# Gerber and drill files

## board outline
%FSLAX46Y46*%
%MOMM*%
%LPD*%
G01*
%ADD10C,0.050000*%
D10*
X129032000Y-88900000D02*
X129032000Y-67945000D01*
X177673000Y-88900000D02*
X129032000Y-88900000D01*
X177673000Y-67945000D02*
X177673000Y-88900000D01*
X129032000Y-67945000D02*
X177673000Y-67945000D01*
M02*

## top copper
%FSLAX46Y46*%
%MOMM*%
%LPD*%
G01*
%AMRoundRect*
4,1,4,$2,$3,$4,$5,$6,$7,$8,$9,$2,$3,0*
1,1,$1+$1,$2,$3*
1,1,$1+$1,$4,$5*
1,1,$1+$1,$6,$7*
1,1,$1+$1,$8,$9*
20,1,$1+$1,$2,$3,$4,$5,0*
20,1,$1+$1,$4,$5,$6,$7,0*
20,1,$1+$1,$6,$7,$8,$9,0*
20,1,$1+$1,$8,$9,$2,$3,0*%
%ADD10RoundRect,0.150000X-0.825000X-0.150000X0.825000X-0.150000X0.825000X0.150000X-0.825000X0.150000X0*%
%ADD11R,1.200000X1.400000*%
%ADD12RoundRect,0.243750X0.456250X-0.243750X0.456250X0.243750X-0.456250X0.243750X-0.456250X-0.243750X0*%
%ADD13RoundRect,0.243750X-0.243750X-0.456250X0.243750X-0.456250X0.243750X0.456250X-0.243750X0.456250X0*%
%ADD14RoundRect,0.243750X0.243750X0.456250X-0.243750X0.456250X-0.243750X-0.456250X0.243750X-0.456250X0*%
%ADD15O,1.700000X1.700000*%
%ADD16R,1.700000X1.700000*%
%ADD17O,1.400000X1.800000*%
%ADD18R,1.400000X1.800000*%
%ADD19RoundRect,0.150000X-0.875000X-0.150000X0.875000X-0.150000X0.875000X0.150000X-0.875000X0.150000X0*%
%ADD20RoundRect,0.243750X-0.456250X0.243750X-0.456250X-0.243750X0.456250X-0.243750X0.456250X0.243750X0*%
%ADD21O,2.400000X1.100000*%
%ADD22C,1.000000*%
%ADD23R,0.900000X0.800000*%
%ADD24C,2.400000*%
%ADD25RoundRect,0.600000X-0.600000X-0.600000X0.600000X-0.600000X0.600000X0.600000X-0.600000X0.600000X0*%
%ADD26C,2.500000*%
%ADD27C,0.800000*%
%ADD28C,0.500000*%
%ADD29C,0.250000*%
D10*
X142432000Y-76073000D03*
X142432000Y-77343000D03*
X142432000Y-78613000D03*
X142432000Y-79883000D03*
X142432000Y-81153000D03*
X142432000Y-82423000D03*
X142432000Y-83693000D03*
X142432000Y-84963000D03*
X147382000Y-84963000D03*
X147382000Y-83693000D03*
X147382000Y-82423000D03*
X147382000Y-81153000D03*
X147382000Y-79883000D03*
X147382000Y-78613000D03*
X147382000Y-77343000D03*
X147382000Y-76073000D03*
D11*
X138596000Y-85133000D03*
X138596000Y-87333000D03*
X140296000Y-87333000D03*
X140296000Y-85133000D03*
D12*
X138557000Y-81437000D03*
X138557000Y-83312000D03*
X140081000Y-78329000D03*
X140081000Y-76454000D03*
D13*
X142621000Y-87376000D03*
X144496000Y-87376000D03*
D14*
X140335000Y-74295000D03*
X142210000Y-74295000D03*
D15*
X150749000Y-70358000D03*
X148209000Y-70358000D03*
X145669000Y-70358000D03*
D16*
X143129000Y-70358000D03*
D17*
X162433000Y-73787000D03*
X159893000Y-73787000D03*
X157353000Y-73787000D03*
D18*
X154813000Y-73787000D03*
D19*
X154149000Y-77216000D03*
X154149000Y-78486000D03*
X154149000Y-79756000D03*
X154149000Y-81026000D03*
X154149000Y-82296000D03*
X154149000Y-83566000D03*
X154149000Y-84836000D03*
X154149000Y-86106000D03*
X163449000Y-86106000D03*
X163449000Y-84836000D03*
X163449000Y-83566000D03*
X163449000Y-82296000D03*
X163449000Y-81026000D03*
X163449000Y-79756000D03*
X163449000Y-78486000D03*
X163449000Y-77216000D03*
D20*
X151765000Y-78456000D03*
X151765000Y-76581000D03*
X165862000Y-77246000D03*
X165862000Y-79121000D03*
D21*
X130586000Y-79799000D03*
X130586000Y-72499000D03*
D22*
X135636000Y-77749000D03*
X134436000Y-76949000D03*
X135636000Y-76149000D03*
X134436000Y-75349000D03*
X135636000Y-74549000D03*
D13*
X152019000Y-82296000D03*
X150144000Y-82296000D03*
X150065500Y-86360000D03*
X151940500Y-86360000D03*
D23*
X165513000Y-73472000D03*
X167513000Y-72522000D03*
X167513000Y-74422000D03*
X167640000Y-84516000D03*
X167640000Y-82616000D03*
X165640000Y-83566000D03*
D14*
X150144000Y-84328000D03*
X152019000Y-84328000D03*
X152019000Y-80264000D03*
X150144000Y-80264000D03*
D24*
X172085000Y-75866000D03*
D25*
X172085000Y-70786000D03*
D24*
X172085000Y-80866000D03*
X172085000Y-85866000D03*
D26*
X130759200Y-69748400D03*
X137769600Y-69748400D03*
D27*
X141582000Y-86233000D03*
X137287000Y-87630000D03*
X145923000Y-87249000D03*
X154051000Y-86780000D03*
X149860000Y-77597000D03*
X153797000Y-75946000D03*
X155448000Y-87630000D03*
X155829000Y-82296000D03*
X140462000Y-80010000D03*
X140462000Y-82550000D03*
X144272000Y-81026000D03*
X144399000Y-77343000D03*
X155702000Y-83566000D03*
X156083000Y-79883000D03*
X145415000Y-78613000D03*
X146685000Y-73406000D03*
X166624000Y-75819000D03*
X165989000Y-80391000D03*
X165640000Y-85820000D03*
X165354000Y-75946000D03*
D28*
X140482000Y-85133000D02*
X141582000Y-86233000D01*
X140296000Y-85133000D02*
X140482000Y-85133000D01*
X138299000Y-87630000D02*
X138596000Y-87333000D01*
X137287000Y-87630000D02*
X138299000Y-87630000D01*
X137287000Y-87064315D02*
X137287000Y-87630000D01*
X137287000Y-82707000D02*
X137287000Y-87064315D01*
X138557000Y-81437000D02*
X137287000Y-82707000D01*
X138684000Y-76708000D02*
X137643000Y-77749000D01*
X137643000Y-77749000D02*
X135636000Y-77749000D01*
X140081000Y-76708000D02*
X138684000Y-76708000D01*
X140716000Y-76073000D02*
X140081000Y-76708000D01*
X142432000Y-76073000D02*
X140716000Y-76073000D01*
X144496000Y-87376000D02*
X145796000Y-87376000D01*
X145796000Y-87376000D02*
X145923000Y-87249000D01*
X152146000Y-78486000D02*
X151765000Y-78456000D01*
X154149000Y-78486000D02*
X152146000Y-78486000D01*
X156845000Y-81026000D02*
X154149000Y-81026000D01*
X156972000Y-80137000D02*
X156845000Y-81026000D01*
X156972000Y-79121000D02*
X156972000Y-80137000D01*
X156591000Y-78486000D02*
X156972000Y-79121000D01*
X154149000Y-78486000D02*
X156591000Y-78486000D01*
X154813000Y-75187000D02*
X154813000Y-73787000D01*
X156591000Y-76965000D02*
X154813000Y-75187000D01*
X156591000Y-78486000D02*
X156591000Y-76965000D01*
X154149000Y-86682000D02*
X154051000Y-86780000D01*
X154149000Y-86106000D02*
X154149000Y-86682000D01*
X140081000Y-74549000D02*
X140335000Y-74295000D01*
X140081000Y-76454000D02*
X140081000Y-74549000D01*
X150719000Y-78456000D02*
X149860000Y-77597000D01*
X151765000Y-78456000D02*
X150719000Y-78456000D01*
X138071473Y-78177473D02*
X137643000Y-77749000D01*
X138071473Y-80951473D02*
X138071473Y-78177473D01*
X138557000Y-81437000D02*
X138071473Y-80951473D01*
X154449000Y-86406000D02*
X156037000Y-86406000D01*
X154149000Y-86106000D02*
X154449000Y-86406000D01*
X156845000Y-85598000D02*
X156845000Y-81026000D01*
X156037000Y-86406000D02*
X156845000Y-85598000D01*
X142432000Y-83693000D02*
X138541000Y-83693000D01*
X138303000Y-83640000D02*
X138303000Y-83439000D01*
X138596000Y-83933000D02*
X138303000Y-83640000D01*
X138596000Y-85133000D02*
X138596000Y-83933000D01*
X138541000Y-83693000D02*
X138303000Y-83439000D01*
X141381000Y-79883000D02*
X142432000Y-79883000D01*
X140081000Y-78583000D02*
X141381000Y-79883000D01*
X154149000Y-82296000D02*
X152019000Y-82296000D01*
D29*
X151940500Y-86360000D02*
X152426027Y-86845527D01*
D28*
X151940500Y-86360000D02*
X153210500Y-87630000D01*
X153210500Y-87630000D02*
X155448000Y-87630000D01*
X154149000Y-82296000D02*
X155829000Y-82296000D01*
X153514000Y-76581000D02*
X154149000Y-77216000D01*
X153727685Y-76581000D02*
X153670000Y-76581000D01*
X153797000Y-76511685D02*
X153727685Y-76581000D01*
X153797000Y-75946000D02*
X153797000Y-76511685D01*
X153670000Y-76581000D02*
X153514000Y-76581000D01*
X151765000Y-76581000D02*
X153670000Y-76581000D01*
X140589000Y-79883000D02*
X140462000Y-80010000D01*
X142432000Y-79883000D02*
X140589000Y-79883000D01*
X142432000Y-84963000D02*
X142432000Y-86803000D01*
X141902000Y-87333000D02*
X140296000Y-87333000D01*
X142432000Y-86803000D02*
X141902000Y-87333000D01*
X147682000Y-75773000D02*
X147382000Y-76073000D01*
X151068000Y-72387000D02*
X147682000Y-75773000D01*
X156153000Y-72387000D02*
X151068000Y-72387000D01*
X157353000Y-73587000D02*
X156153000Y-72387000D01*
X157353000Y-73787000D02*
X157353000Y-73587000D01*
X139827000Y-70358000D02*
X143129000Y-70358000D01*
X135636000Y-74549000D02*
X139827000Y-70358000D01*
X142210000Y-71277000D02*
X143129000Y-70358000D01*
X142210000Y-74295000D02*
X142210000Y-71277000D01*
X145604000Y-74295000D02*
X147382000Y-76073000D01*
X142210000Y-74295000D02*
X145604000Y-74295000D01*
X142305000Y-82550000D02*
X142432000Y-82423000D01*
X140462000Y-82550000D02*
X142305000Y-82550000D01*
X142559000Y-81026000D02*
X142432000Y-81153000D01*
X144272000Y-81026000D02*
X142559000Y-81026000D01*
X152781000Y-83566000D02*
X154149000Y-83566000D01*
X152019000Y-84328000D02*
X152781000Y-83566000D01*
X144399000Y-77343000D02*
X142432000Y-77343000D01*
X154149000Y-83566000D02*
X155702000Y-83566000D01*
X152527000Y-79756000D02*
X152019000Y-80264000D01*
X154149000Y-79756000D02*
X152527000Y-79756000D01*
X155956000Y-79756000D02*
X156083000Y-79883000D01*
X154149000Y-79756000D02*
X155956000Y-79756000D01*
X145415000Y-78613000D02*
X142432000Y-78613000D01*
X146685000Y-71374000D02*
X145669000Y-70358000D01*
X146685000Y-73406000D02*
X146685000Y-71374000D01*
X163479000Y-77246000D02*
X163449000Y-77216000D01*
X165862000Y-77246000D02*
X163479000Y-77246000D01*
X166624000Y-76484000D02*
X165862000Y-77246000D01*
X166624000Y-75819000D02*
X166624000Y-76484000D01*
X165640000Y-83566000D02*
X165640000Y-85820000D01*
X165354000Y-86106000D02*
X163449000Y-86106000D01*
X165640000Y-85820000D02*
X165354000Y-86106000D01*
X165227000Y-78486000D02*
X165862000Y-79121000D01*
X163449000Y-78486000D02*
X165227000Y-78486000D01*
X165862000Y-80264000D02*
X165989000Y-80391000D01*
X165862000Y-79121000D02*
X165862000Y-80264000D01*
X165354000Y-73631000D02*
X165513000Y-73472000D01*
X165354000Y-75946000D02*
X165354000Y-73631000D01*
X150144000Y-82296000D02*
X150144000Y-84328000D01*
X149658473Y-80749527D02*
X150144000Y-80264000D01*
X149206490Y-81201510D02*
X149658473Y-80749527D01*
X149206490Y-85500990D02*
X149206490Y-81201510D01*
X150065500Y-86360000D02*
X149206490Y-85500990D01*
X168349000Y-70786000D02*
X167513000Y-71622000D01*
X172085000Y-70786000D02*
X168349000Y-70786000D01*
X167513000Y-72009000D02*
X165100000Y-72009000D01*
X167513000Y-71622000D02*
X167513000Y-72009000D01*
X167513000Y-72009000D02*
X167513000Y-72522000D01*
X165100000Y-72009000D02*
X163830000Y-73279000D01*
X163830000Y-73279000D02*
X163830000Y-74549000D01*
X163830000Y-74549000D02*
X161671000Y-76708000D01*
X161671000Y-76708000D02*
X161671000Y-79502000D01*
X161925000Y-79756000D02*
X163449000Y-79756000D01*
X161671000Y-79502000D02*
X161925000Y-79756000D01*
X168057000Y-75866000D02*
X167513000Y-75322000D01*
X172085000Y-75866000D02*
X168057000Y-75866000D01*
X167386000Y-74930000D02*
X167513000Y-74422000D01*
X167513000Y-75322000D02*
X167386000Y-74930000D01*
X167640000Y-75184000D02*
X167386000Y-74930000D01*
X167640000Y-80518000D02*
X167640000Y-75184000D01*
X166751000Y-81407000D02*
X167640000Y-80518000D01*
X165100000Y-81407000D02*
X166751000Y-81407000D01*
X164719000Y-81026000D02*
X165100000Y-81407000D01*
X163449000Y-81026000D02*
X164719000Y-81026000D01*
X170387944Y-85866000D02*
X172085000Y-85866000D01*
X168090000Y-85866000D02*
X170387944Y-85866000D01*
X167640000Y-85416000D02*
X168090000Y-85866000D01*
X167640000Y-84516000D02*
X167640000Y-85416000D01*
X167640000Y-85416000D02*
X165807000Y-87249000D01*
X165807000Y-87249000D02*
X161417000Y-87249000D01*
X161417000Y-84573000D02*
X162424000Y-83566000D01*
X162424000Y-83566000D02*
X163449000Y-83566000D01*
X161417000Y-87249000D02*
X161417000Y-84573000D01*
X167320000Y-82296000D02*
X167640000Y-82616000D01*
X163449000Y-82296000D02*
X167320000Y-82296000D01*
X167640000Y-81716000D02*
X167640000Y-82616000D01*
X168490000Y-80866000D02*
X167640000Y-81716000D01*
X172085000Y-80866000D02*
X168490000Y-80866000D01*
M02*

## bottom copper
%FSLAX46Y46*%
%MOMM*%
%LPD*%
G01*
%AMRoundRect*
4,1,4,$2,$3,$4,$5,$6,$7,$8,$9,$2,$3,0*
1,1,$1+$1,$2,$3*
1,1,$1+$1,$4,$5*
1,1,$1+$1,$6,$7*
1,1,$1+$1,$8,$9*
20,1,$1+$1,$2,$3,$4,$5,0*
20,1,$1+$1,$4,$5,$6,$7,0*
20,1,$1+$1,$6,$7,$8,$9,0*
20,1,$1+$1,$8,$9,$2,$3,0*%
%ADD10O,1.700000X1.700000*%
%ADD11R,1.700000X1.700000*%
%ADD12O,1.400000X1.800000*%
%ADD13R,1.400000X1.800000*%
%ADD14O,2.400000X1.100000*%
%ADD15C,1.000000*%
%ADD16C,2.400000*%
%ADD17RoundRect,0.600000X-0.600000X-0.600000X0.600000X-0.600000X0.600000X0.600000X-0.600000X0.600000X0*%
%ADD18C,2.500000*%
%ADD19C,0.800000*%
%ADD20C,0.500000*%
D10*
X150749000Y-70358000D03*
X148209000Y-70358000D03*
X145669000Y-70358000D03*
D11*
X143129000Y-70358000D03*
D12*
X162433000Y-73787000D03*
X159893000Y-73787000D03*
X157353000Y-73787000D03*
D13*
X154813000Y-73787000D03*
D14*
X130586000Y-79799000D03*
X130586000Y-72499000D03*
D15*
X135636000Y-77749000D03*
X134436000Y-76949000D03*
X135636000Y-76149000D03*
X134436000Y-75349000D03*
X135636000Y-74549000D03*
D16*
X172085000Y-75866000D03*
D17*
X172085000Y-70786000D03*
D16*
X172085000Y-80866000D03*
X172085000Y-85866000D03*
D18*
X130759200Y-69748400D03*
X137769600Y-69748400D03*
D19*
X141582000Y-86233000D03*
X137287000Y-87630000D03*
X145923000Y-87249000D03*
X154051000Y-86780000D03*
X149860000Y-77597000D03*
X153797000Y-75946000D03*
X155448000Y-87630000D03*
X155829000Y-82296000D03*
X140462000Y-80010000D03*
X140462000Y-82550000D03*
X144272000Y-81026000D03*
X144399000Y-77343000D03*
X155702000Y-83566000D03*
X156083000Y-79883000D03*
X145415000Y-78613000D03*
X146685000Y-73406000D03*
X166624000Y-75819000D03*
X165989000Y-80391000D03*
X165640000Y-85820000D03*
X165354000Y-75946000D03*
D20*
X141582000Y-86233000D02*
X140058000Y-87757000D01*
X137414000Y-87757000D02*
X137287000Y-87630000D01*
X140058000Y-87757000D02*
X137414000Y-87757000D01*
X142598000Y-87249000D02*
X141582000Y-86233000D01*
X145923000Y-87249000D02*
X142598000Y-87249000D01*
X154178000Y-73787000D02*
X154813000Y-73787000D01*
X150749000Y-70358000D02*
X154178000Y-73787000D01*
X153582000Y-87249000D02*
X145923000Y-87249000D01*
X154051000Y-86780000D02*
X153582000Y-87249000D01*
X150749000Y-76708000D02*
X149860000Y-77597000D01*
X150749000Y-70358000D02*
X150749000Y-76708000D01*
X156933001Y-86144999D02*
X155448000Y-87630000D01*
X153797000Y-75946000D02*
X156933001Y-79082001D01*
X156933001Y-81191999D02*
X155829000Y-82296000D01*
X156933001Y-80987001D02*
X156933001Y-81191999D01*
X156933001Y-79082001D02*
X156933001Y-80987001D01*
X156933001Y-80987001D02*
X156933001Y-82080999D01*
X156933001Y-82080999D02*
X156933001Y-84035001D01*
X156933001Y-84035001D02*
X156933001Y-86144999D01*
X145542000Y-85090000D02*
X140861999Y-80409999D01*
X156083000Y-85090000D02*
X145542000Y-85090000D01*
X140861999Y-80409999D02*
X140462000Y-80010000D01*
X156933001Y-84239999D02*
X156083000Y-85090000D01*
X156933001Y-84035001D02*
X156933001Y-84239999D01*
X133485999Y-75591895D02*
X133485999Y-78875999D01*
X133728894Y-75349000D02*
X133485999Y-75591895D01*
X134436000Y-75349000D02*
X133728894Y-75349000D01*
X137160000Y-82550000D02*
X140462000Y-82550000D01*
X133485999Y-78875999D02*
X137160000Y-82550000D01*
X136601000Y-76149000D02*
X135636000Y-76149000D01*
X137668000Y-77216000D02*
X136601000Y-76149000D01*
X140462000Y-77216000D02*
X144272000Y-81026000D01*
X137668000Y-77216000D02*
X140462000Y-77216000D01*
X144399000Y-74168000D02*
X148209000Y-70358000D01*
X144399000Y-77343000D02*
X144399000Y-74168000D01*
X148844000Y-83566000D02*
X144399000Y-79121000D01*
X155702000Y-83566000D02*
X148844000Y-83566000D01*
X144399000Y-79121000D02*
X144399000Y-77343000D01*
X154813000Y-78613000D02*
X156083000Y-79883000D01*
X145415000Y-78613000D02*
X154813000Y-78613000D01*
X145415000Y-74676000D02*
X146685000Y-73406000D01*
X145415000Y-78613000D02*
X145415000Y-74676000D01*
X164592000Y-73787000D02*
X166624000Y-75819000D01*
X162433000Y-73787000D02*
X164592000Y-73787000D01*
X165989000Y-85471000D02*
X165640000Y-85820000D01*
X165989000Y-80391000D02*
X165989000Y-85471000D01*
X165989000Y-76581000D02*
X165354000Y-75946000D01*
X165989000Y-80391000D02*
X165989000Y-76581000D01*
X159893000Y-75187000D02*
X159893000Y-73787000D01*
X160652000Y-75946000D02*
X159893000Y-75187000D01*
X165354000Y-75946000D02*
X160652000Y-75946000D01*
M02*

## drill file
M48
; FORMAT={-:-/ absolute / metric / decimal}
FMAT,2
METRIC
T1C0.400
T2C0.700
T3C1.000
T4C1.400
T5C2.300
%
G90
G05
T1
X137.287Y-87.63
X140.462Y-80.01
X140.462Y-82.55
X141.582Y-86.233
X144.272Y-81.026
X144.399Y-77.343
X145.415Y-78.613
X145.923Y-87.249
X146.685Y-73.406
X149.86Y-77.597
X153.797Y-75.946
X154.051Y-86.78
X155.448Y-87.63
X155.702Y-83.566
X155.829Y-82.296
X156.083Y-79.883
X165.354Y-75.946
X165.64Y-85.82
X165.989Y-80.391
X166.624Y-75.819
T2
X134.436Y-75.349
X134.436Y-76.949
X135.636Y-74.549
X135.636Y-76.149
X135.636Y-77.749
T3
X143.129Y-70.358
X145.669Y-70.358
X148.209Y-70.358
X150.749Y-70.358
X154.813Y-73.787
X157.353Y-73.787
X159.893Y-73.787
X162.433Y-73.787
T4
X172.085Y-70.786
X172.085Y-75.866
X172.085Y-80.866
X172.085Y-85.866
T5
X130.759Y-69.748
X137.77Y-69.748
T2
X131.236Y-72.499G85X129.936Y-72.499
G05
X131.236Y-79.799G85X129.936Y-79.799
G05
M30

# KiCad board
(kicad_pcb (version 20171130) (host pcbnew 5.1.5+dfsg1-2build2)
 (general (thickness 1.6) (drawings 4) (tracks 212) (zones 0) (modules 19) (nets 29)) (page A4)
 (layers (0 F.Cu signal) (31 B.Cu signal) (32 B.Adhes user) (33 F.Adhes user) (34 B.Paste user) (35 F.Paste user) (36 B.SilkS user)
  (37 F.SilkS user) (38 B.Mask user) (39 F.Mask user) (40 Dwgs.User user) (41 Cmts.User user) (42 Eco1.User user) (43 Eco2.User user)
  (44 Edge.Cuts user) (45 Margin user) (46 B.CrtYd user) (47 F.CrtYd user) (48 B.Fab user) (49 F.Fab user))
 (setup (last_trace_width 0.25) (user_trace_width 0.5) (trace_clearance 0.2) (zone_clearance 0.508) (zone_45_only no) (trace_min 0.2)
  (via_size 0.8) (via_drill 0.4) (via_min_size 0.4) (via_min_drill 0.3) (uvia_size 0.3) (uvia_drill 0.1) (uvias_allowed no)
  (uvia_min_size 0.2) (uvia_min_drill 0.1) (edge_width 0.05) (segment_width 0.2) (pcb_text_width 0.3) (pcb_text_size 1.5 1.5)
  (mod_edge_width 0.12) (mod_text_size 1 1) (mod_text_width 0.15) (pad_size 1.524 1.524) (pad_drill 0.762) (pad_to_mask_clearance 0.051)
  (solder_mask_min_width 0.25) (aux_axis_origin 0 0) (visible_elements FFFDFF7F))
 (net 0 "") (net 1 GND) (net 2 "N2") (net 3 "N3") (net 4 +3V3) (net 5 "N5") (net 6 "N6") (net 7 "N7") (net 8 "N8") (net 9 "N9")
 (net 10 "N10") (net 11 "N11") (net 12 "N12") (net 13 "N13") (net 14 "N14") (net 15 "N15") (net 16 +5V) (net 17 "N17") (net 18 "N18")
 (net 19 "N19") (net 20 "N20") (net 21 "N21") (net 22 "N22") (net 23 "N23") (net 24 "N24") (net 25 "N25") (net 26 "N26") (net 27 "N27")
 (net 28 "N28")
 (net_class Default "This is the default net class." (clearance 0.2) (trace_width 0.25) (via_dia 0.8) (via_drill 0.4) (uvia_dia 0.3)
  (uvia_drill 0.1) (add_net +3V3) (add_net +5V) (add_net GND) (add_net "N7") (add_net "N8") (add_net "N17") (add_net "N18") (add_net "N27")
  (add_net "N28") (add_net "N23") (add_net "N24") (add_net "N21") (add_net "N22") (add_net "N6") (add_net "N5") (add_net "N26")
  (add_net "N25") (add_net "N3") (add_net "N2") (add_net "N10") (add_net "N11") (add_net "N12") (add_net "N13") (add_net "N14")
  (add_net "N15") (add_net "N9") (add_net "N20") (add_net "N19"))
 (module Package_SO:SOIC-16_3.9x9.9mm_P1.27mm (layer F.Cu) (at 144.907 80.518)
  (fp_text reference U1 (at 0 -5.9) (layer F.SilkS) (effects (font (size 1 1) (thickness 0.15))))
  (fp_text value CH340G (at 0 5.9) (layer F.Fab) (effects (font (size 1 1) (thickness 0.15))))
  (pad 1 smd roundrect (at -2.475 -4.445) (size 1.95 0.6) (layers F.Cu F.Paste F.Mask) (roundrect_rratio 0.25) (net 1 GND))
  (pad 2 smd roundrect (at -2.475 -3.175) (size 1.95 0.6) (layers F.Cu F.Paste F.Mask) (roundrect_rratio 0.25) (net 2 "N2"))
  (pad 3 smd roundrect (at -2.475 -1.905) (size 1.95 0.6) (layers F.Cu F.Paste F.Mask) (roundrect_rratio 0.25) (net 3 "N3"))
  (pad 4 smd roundrect (at -2.475 -0.635) (size 1.95 0.6) (layers F.Cu F.Paste F.Mask) (roundrect_rratio 0.25) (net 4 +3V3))
  (pad 5 smd roundrect (at -2.475 0.635) (size 1.95 0.6) (layers F.Cu F.Paste F.Mask) (roundrect_rratio 0.25) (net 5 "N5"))
  (pad 6 smd roundrect (at -2.475 1.905) (size 1.95 0.6) (layers F.Cu F.Paste F.Mask) (roundrect_rratio 0.25) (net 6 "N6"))
  (pad 7 smd roundrect (at -2.475 3.175) (size 1.95 0.6) (layers F.Cu F.Paste F.Mask) (roundrect_rratio 0.25) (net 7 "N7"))
  (pad 8 smd roundrect (at -2.475 4.445) (size 1.95 0.6) (layers F.Cu F.Paste F.Mask) (roundrect_rratio 0.25) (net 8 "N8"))
  (pad 9 smd roundrect (at 2.475 4.445) (size 1.95 0.6) (layers F.Cu F.Paste F.Mask) (roundrect_rratio 0.25) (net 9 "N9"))
  (pad 10 smd roundrect (at 2.475 3.175) (size 1.95 0.6) (layers F.Cu F.Paste F.Mask) (roundrect_rratio 0.25) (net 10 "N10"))
  (pad 11 smd roundrect (at 2.475 1.905) (size 1.95 0.6) (layers F.Cu F.Paste F.Mask) (roundrect_rratio 0.25) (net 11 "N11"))
  (pad 12 smd roundrect (at 2.475 0.635) (size 1.95 0.6) (layers F.Cu F.Paste F.Mask) (roundrect_rratio 0.25) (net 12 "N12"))
  (pad 13 smd roundrect (at 2.475 -0.635) (size 1.95 0.6) (layers F.Cu F.Paste F.Mask) (roundrect_rratio 0.25) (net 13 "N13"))
  (pad 14 smd roundrect (at 2.475 -1.905) (size 1.95 0.6) (layers F.Cu F.Paste F.Mask) (roundrect_rratio 0.25) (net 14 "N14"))
  (pad 15 smd roundrect (at 2.475 -3.175) (size 1.95 0.6) (layers F.Cu F.Paste F.Mask) (roundrect_rratio 0.25) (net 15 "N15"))
  (pad 16 smd roundrect (at 2.475 -4.445) (size 1.95 0.6) (layers F.Cu F.Paste F.Mask) (roundrect_rratio 0.25) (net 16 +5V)))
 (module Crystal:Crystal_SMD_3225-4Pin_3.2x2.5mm (layer F.Cu) (at 139.446 86.233 270)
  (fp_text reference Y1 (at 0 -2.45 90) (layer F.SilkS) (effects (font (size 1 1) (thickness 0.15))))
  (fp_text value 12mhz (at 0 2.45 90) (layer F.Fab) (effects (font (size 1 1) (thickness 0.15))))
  (pad 1 smd rect (at -1.1 0.85 270) (size 1.4 1.2) (layers F.Cu F.Paste F.Mask) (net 7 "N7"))
  (pad 2 smd rect (at 1.1 0.85 270) (size 1.4 1.2) (layers F.Cu F.Paste F.Mask) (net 1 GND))
  (pad 3 smd rect (at 1.1 -0.85 270) (size 1.4 1.2) (layers F.Cu F.Paste F.Mask) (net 8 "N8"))
  (pad 4 smd rect (at -1.1 -0.85 270) (size 1.4 1.2) (layers F.Cu F.Paste F.Mask) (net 1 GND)))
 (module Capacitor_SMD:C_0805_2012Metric (layer F.Cu) (at 138.557 82.3745 90)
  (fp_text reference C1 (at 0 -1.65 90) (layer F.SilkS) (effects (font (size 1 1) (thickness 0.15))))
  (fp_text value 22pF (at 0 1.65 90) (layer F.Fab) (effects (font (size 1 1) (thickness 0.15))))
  (pad 2 smd roundrect (at 0.9375 0 90) (size 0.975 1.4) (layers F.Cu F.Paste F.Mask) (roundrect_rratio 0.25) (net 1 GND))
  (pad 1 smd roundrect (at -0.9375 0 90) (size 0.975 1.4) (layers F.Cu F.Paste F.Mask) (roundrect_rratio 0.25) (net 7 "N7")))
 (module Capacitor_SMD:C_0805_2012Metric (layer F.Cu) (at 140.081 77.3915 90)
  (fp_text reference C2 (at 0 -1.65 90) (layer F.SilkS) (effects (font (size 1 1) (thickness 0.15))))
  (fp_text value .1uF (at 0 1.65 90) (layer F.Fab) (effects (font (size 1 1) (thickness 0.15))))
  (pad 1 smd roundrect (at -0.9375 0 90) (size 0.975 1.4) (layers F.Cu F.Paste F.Mask) (roundrect_rratio 0.25) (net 4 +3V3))
  (pad 2 smd roundrect (at 0.9375 0 90) (size 0.975 1.4) (layers F.Cu F.Paste F.Mask) (roundrect_rratio 0.25) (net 1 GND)))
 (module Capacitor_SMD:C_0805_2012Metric (layer F.Cu) (at 143.5585 87.376)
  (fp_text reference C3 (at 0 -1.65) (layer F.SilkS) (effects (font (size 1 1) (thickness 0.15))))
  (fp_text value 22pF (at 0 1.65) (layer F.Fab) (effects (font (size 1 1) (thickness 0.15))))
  (pad 1 smd roundrect (at -0.9375 0) (size 0.975 1.4) (layers F.Cu F.Paste F.Mask) (roundrect_rratio 0.25) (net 8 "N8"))
  (pad 2 smd roundrect (at 0.9375 0) (size 0.975 1.4) (layers F.Cu F.Paste F.Mask) (roundrect_rratio 0.25) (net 1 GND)))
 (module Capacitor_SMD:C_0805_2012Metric (layer F.Cu) (at 141.2725 74.295 180)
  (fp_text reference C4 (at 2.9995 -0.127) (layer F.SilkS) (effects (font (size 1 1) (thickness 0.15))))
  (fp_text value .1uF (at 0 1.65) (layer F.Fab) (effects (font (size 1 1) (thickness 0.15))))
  (pad 2 smd roundrect (at 0.9375 0 180) (size 0.975 1.4) (layers F.Cu F.Paste F.Mask) (roundrect_rratio 0.25) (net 1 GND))
  (pad 1 smd roundrect (at -0.9375 0 180) (size 0.975 1.4) (layers F.Cu F.Paste F.Mask) (roundrect_rratio 0.25) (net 16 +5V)))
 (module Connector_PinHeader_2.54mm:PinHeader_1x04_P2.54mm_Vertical (layer F.Cu) (at 143.129 70.358 90)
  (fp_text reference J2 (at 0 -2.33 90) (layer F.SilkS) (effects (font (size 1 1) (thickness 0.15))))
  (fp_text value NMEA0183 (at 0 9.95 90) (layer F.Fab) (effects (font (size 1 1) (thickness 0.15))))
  (pad 4 thru_hole oval (at 0 7.62 90) (size 1.7 1.7) (drill 1) (layers *.Cu *.Mask) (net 1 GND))
  (pad 3 thru_hole oval (at 0 5.08 90) (size 1.7 1.7) (drill 1) (layers *.Cu *.Mask) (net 2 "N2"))
  (pad 2 thru_hole oval (at 0 2.54 90) (size 1.7 1.7) (drill 1) (layers *.Cu *.Mask) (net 3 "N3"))
  (pad 1 thru_hole rect (at 0 0 90) (size 1.7 1.7) (drill 1) (layers *.Cu *.Mask) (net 16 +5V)))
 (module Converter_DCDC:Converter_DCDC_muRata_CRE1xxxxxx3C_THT (layer F.Cu) (at 154.813 73.787 90)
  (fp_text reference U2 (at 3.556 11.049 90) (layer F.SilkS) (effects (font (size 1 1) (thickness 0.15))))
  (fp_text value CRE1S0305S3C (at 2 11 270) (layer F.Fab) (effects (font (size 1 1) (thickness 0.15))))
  (pad 4 thru_hole oval (at 0 7.62) (size 1.4 1.8) (drill 1) (layers *.Cu *.Mask) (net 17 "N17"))
  (pad 3 thru_hole oval (at 0 5.08) (size 1.4 1.8) (drill 1) (layers *.Cu *.Mask) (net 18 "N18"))
  (pad 2 thru_hole oval (at 0 2.54) (size 1.4 1.8) (drill 1) (layers *.Cu *.Mask) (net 16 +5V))
  (pad 1 thru_hole rect (at 0 0) (size 1.4 1.8) (drill 1) (layers *.Cu *.Mask) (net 1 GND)))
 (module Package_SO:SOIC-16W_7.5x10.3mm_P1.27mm (layer F.Cu) (at 158.799 81.661)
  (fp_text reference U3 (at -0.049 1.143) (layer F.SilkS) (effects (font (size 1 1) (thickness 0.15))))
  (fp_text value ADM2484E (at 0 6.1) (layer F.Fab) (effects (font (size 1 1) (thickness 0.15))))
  (pad 1 smd roundrect (at -4.65 -4.445) (size 2.05 0.6) (layers F.Cu F.Paste F.Mask) (roundrect_rratio 0.25) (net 4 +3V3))
  (pad 2 smd roundrect (at -4.65 -3.175) (size 2.05 0.6) (layers F.Cu F.Paste F.Mask) (roundrect_rratio 0.25) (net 1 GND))
  (pad 3 smd roundrect (at -4.65 -1.905) (size 2.05 0.6) (layers F.Cu F.Paste F.Mask) (roundrect_rratio 0.25) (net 3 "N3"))
  (pad 4 smd roundrect (at -4.65 -0.635) (size 2.05 0.6) (layers F.Cu F.Paste F.Mask) (roundrect_rratio 0.25) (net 1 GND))
  (pad 5 smd roundrect (at -4.65 0.635) (size 2.05 0.6) (layers F.Cu F.Paste F.Mask) (roundrect_rratio 0.25) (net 4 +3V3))
  (pad 6 smd roundrect (at -4.65 1.905) (size 2.05 0.6) (layers F.Cu F.Paste F.Mask) (roundrect_rratio 0.25) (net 2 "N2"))
  (pad 7 smd roundrect (at -4.65 3.175) (size 2.05 0.6) (layers F.Cu F.Paste F.Mask) (roundrect_rratio 0.25) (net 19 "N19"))
  (pad 8 smd roundrect (at -4.65 4.445) (size 2.05 0.6) (layers F.Cu F.Paste F.Mask) (roundrect_rratio 0.25) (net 1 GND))
  (pad 9 smd roundrect (at 4.65 4.445) (size 2.05 0.6) (layers F.Cu F.Paste F.Mask) (roundrect_rratio 0.25) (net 18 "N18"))
  (pad 10 smd roundrect (at 4.65 3.175) (size 2.05 0.6) (layers F.Cu F.Paste F.Mask) (roundrect_rratio 0.25) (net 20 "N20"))
  (pad 11 smd roundrect (at 4.65 1.905) (size 2.05 0.6) (layers F.Cu F.Paste F.Mask) (roundrect_rratio 0.25) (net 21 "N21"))
  (pad 12 smd roundrect (at 4.65 0.635) (size 2.05 0.6) (layers F.Cu F.Paste F.Mask) (roundrect_rratio 0.25) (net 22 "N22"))
  (pad 13 smd roundrect (at 4.65 -0.635) (size 2.05 0.6) (layers F.Cu F.Paste F.Mask) (roundrect_rratio 0.25) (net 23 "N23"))
  (pad 14 smd roundrect (at 4.65 -1.905) (size 2.05 0.6) (layers F.Cu F.Paste F.Mask) (roundrect_rratio 0.25) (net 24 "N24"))
  (pad 15 smd roundrect (at 4.65 -3.175) (size 2.05 0.6) (layers F.Cu F.Paste F.Mask) (roundrect_rratio 0.25) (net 18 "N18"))
  (pad 16 smd roundrect (at 4.65 -4.445) (size 2.05 0.6) (layers F.Cu F.Paste F.Mask) (roundrect_rratio 0.25) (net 17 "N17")))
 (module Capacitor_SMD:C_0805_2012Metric (layer F.Cu) (at 151.765 77.5185 270)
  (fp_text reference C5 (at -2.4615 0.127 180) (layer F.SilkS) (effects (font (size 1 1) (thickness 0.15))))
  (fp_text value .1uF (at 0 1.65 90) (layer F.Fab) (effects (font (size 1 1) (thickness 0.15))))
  (pad 2 smd roundrect (at 0.9375 0 270) (size 0.975 1.4) (layers F.Cu F.Paste F.Mask) (roundrect_rratio 0.25) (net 1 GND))
  (pad 1 smd roundrect (at -0.9375 0 270) (size 0.975 1.4) (layers F.Cu F.Paste F.Mask) (roundrect_rratio 0.25) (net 4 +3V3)))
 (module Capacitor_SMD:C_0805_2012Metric (layer F.Cu) (at 165.862 78.1835 270)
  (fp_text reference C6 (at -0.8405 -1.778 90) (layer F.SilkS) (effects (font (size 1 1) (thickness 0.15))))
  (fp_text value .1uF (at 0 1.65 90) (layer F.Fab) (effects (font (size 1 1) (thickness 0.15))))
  (pad 1 smd roundrect (at -0.9375 0 270) (size 0.975 1.4) (layers F.Cu F.Paste F.Mask) (roundrect_rratio 0.25) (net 17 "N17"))
  (pad 2 smd roundrect (at 0.9375 0 270) (size 0.975 1.4) (layers F.Cu F.Paste F.Mask) (roundrect_rratio 0.25) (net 18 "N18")))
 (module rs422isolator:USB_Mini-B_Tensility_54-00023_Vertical (layer F.Cu) (at 135.636 74.549 270)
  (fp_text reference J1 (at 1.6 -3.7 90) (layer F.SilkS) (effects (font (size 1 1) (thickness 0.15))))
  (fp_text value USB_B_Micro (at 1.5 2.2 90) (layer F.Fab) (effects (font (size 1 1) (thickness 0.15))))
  (pad 6 thru_hole oval (at 5.25 5.05 270) (size 1.1 2.4) (drill oval 0.7 2) (layers *.Cu *.Mask) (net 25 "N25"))
  (pad 6 thru_hole oval (at -2.05 5.05 270) (size 1.1 2.4) (drill oval 0.7 2) (layers *.Cu *.Mask) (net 25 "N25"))
  (pad 5 thru_hole circle (at 3.2 0 270) (size 1 1) (drill 0.7) (layers *.Cu *.Mask) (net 1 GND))
  (pad 4 thru_hole circle (at 2.4 1.2 270) (size 1 1) (drill 0.7) (layers *.Cu *.Mask) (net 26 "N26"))
  (pad 3 thru_hole circle (at 1.6 0 270) (size 1 1) (drill 0.7) (layers *.Cu *.Mask) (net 5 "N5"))
  (pad 2 thru_hole circle (at 0.8 1.2 270) (size 1 1) (drill 0.7) (layers *.Cu *.Mask) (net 6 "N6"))
  (pad 1 thru_hole circle (at 0 0 270) (size 1 1) (drill 0.7) (layers *.Cu *.Mask) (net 16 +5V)))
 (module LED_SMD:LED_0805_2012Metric (layer F.Cu) (at 151.0815 82.296)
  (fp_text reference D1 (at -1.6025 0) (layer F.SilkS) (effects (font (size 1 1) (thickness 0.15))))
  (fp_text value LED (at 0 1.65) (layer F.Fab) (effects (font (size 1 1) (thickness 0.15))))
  (pad 2 smd roundrect (at 0.9375 0) (size 0.975 1.4) (layers F.Cu F.Paste F.Mask) (roundrect_rratio 0.25) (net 4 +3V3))
  (pad 1 smd roundrect (at -0.9375 0) (size 0.975 1.4) (layers F.Cu F.Paste F.Mask) (roundrect_rratio 0.25) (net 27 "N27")))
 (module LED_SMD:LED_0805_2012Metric (layer F.Cu) (at 151.003 86.36)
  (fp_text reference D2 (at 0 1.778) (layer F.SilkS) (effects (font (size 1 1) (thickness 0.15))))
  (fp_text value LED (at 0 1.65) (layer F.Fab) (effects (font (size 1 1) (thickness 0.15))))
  (pad 1 smd roundrect (at -0.9375 0) (size 0.975 1.4) (layers F.Cu F.Paste F.Mask) (roundrect_rratio 0.25) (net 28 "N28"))
  (pad 2 smd roundrect (at 0.9375 0) (size 0.975 1.4) (layers F.Cu F.Paste F.Mask) (roundrect_rratio 0.25) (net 4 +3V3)))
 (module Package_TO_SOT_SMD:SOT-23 (layer F.Cu) (at 166.513 73.472 180)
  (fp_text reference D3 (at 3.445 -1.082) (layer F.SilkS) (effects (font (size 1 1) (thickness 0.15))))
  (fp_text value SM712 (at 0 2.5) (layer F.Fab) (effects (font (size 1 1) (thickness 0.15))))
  (pad 3 smd rect (at 1 0 180) (size 0.9 0.8) (layers F.Cu F.Paste F.Mask) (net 18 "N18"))
  (pad 2 smd rect (at -1 0.95 180) (size 0.9 0.8) (layers F.Cu F.Paste F.Mask) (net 24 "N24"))
  (pad 1 smd rect (at -1 -0.95 180) (size 0.9 0.8) (layers F.Cu F.Paste F.Mask) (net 23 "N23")))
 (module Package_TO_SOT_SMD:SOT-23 (layer F.Cu) (at 166.64 83.566 180)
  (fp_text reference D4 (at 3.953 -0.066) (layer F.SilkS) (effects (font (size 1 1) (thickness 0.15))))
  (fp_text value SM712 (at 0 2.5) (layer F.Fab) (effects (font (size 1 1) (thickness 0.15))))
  (pad 1 smd rect (at -1 -0.95 180) (size 0.9 0.8) (layers F.Cu F.Paste F.Mask) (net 21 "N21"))
  (pad 2 smd rect (at -1 0.95 180) (size 0.9 0.8) (layers F.Cu F.Paste F.Mask) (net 22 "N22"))
  (pad 3 smd rect (at 1 0 180) (size 0.9 0.8) (layers F.Cu F.Paste F.Mask) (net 18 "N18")))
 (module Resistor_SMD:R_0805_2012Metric (layer F.Cu) (at 151.0815 84.328 180)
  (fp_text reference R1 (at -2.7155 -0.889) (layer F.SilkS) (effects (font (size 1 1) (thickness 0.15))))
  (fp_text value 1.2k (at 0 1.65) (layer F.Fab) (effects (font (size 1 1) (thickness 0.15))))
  (pad 2 smd roundrect (at 0.9375 0 180) (size 0.975 1.4) (layers F.Cu F.Paste F.Mask) (roundrect_rratio 0.25) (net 27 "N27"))
  (pad 1 smd roundrect (at -0.9375 0 180) (size 0.975 1.4) (layers F.Cu F.Paste F.Mask) (roundrect_rratio 0.25) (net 2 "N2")))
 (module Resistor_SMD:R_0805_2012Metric (layer F.Cu) (at 151.0815 80.264 180)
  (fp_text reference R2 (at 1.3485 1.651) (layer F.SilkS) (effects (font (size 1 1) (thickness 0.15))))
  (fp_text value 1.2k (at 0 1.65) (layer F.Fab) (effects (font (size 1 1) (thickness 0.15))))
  (pad 1 smd roundrect (at -0.9375 0 180) (size 0.975 1.4) (layers F.Cu F.Paste F.Mask) (roundrect_rratio 0.25) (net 3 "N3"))
  (pad 2 smd roundrect (at 0.9375 0 180) (size 0.975 1.4) (layers F.Cu F.Paste F.Mask) (roundrect_rratio 0.25) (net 28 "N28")))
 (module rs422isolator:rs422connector (layer F.Cu) (at 172.085 70.866)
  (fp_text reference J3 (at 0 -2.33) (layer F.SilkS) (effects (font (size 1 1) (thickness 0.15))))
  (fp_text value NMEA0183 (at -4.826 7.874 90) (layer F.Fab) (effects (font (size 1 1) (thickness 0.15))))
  (pad 2 thru_hole circle (at 0 5) (size 2.4 2.4) (drill 1.4) (layers *.Cu *.Mask) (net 23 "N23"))
  (pad 1 thru_hole roundrect (at 0 -0.08) (size 2.4 2.4) (drill 1.4) (layers *.Cu *.Mask) (roundrect_rratio 0.25) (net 24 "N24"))
  (pad 3 thru_hole circle (at 0 10) (size 2.4 2.4) (drill 1.4) (layers *.Cu *.Mask) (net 22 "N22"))
  (pad 4 thru_hole circle (at 0 15) (size 2.4 2.4) (drill 1.4) (layers *.Cu *.Mask) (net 21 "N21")))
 (gr_line (start 129.032 88.9) (end 129.032 67.945) (layer Edge.Cuts) (width 0.05))
 (gr_line (start 177.673 88.9) (end 129.032 88.9) (layer Edge.Cuts) (width 0.05))
 (gr_line (start 177.673 67.945) (end 177.673 88.9) (layer Edge.Cuts) (width 0.05))
 (gr_line (start 129.032 67.945) (end 177.673 67.945) (layer Edge.Cuts) (width 0.05))
 (via (at 130.7592 69.7484) (size 2.5) (drill 2.3) (layers F.Cu B.Cu) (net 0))
 (via (at 137.7696 69.7484) (size 2.5) (drill 2.3) (layers F.Cu B.Cu) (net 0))
 (via (at 141.582 86.233) (size 0.8) (drill 0.4) (layers F.Cu B.Cu) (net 1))
 (segment (start 140.482 85.133) (end 141.582 86.233) (width 0.5) (layer F.Cu) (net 1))
 (segment (start 140.296 85.133) (end 140.482 85.133) (width 0.5) (layer F.Cu) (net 1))
 (segment (start 141.582 86.233) (end 140.058 87.757) (width 0.5) (layer B.Cu) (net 1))
 (via (at 137.287 87.63) (size 0.8) (drill 0.4) (layers F.Cu B.Cu) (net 1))
 (segment (start 137.414 87.757) (end 137.287 87.63) (width 0.5) (layer B.Cu) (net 1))
 (segment (start 140.058 87.757) (end 137.414 87.757) (width 0.5) (layer B.Cu) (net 1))
 (segment (start 138.299 87.63) (end 138.596 87.333) (width 0.5) (layer F.Cu) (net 1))
 (segment (start 137.287 87.63) (end 138.299 87.63) (width 0.5) (layer F.Cu) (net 1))
 (segment (start 137.287 87.064315) (end 137.287 87.63) (width 0.5) (layer F.Cu) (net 1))
 (segment (start 137.287 82.707) (end 137.287 87.064315) (width 0.5) (layer F.Cu) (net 1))
 (segment (start 138.557 81.437) (end 137.287 82.707) (width 0.5) (layer F.Cu) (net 1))
 (segment (start 138.684 76.708) (end 137.643 77.749) (width 0.5) (layer F.Cu) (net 1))
 (segment (start 137.643 77.749) (end 135.636 77.749) (width 0.5) (layer F.Cu) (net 1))
 (segment (start 140.081 76.708) (end 138.684 76.708) (width 0.5) (layer F.Cu) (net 1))
 (segment (start 140.716 76.073) (end 140.081 76.708) (width 0.5) (layer F.Cu) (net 1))
 (segment (start 142.432 76.073) (end 140.716 76.073) (width 0.5) (layer F.Cu) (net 1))
 (segment (start 142.598 87.249) (end 141.582 86.233) (width 0.5) (layer B.Cu) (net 1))
 (via (at 145.923 87.249) (size 0.8) (drill 0.4) (layers F.Cu B.Cu) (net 1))
 (segment (start 144.496 87.376) (end 145.796 87.376) (width 0.5) (layer F.Cu) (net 1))
 (segment (start 145.923 87.249) (end 142.598 87.249) (width 0.5) (layer B.Cu) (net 1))
 (segment (start 145.796 87.376) (end 145.923 87.249) (width 0.5) (layer F.Cu) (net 1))
 (segment (start 152.146 78.486) (end 151.765 78.456) (width 0.5) (layer F.Cu) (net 1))
 (segment (start 154.149 78.486) (end 152.146 78.486) (width 0.5) (layer F.Cu) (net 1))
 (segment (start 156.845 81.026) (end 154.149 81.026) (width 0.5) (layer F.Cu) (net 1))
 (segment (start 156.972 80.137) (end 156.845 81.026) (width 0.5) (layer F.Cu) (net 1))
 (segment (start 156.972 79.121) (end 156.972 80.137) (width 0.5) (layer F.Cu) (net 1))
 (segment (start 156.591 78.486) (end 156.972 79.121) (width 0.5) (layer F.Cu) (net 1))
 (segment (start 154.149 78.486) (end 156.591 78.486) (width 0.5) (layer F.Cu) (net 1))
 (segment (start 154.813 75.187) (end 154.813 73.787) (width 0.5) (layer F.Cu) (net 1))
 (segment (start 156.591 76.965) (end 154.813 75.187) (width 0.5) (layer F.Cu) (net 1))
 (segment (start 156.591 78.486) (end 156.591 76.965) (width 0.5) (layer F.Cu) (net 1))
 (segment (start 154.178 73.787) (end 154.813 73.787) (width 0.5) (layer B.Cu) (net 1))
 (segment (start 150.749 70.358) (end 154.178 73.787) (width 0.5) (layer B.Cu) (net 1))
 (via (at 154.051 86.78) (size 0.8) (drill 0.4) (layers F.Cu B.Cu) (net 1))
 (segment (start 154.149 86.682) (end 154.051 86.78) (width 0.5) (layer F.Cu) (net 1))
 (segment (start 154.149 86.106) (end 154.149 86.682) (width 0.5) (layer F.Cu) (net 1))
 (segment (start 153.582 87.249) (end 145.923 87.249) (width 0.5) (layer B.Cu) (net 1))
 (segment (start 154.051 86.78) (end 153.582 87.249) (width 0.5) (layer B.Cu) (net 1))
 (segment (start 140.081 74.549) (end 140.335 74.295) (width 0.5) (layer F.Cu) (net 1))
 (segment (start 140.081 76.454) (end 140.081 74.549) (width 0.5) (layer F.Cu) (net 1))
 (via (at 149.86 77.597) (size 0.8) (drill 0.4) (layers F.Cu B.Cu) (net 1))
 (segment (start 150.749 76.708) (end 149.86 77.597) (width 0.5) (layer B.Cu) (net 1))
 (segment (start 150.749 70.358) (end 150.749 76.708) (width 0.5) (layer B.Cu) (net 1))
 (segment (start 150.719 78.456) (end 149.86 77.597) (width 0.5) (layer F.Cu) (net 1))
 (segment (start 151.765 78.456) (end 150.719 78.456) (width 0.5) (layer F.Cu) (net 1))
 (segment (start 138.071473 78.177473) (end 137.643 77.749) (width 0.5) (layer F.Cu) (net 1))
 (segment (start 138.071473 80.951473) (end 138.071473 78.177473) (width 0.5) (layer F.Cu) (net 1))
 (segment (start 138.557 81.437) (end 138.071473 80.951473) (width 0.5) (layer F.Cu) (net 1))
 (segment (start 154.449 86.406) (end 156.037 86.406) (width 0.5) (layer F.Cu) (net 1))
 (segment (start 154.149 86.106) (end 154.449 86.406) (width 0.5) (layer F.Cu) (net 1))
 (segment (start 156.845 85.598) (end 156.845 81.026) (width 0.5) (layer F.Cu) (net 1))
 (segment (start 156.037 86.406) (end 156.845 85.598) (width 0.5) (layer F.Cu) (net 1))
 (segment (start 142.432 83.693) (end 138.541 83.693) (width 0.5) (layer F.Cu) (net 7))
 (segment (start 138.303 83.64) (end 138.303 83.439) (width 0.5) (layer F.Cu) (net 7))
 (segment (start 138.596 83.933) (end 138.303 83.64) (width 0.5) (layer F.Cu) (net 7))
 (segment (start 138.596 85.133) (end 138.596 83.933) (width 0.5) (layer F.Cu) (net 7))
 (segment (start 138.541 83.693) (end 138.303 83.439) (width 0.5) (layer F.Cu) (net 7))
 (segment (start 141.381 79.883) (end 142.432 79.883) (width 0.5) (layer F.Cu) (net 4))
 (segment (start 140.081 78.583) (end 141.381 79.883) (width 0.5) (layer F.Cu) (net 4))
 (segment (start 154.149 82.296) (end 152.019 82.296) (width 0.5) (layer F.Cu) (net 4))
 (segment (start 151.9405 86.36) (end 152.426027 86.845527) (width 0.25) (layer F.Cu) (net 4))
 (segment (start 151.9405 86.36) (end 153.2105 87.63) (width 0.5) (layer F.Cu) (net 4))
 (segment (start 153.2105 87.63) (end 155.448 87.63) (width 0.5) (layer F.Cu) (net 4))
 (via (at 153.797 75.946) (size 0.8) (drill 0.4) (layers F.Cu B.Cu) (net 4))
 (via (at 155.448 87.63) (size 0.8) (drill 0.4) (layers F.Cu B.Cu) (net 4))
 (segment (start 156.933001 86.144999) (end 155.448 87.63) (width 0.5) (layer B.Cu) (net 4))
 (segment (start 153.797 75.946) (end 156.933001 79.082001) (width 0.5) (layer B.Cu) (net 4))
 (via (at 155.829 82.296) (size 0.8) (drill 0.4) (layers F.Cu B.Cu) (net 4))
 (segment (start 154.149 82.296) (end 155.829 82.296) (width 0.5) (layer F.Cu) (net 4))
 (segment (start 156.933001 81.191999) (end 155.829 82.296) (width 0.5) (layer B.Cu) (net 4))
 (segment (start 156.933001 80.987001) (end 156.933001 81.191999) (width 0.5) (layer B.Cu) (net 4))
 (segment (start 156.933001 79.082001) (end 156.933001 80.987001) (width 0.5) (layer B.Cu) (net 4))
 (segment (start 156.933001 80.987001) (end 156.933001 82.080999) (width 0.5) (layer B.Cu) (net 4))
 (segment (start 153.514 76.581) (end 154.149 77.216) (width 0.5) (layer F.Cu) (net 4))
 (segment (start 153.727685 76.581) (end 153.67 76.581) (width 0.5) (layer F.Cu) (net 4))
 (segment (start 153.797 76.511685) (end 153.727685 76.581) (width 0.5) (layer F.Cu) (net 4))
 (segment (start 153.797 75.946) (end 153.797 76.511685) (width 0.5) (layer F.Cu) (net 4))
 (segment (start 153.67 76.581) (end 153.514 76.581) (width 0.5) (layer F.Cu) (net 4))
 (segment (start 151.765 76.581) (end 153.67 76.581) (width 0.5) (layer F.Cu) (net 4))
 (via (at 140.462 80.01) (size 0.8) (drill 0.4) (layers F.Cu B.Cu) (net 4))
 (segment (start 140.589 79.883) (end 140.462 80.01) (width 0.5) (layer F.Cu) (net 4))
 (segment (start 142.432 79.883) (end 140.589 79.883) (width 0.5) (layer F.Cu) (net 4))
 (segment (start 156.933001 82.080999) (end 156.933001 84.035001) (width 0.5) (layer B.Cu) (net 4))
 (segment (start 156.933001 84.035001) (end 156.933001 86.144999) (width 0.5) (layer B.Cu) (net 4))
 (segment (start 145.542 85.09) (end 140.861999 80.409999) (width 0.5) (layer B.Cu) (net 4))
 (segment (start 156.083 85.09) (end 145.542 85.09) (width 0.5) (layer B.Cu) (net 4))
 (segment (start 140.861999 80.409999) (end 140.462 80.01) (width 0.5) (layer B.Cu) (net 4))
 (segment (start 156.933001 84.239999) (end 156.083 85.09) (width 0.5) (layer B.Cu) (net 4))
 (segment (start 156.933001 84.035001) (end 156.933001 84.239999) (width 0.5) (layer B.Cu) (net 4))
 (segment (start 142.432 84.963) (end 142.432 86.803) (width 0.5) (layer F.Cu) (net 8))
 (segment (start 141.902 87.333) (end 140.296 87.333) (width 0.5) (layer F.Cu) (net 8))
 (segment (start 142.432 86.803) (end 141.902 87.333) (width 0.5) (layer F.Cu) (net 8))
 (segment (start 147.682 75.773) (end 147.382 76.073) (width 0.5) (layer F.Cu) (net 16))
 (segment (start 151.068 72.387) (end 147.682 75.773) (width 0.5) (layer F.Cu) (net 16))
 (segment (start 156.153 72.387) (end 151.068 72.387) (width 0.5) (layer F.Cu) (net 16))
 (segment (start 157.353 73.587) (end 156.153 72.387) (width 0.5) (layer F.Cu) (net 16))
 (segment (start 157.353 73.787) (end 157.353 73.587) (width 0.5) (layer F.Cu) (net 16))
 (segment (start 139.827 70.358) (end 143.129 70.358) (width 0.5) (layer F.Cu) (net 16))
 (segment (start 135.636 74.549) (end 139.827 70.358) (width 0.5) (layer F.Cu) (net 16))
 (segment (start 142.21 71.277) (end 143.129 70.358) (width 0.5) (layer F.Cu) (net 16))
 (segment (start 142.21 74.295) (end 142.21 71.277) (width 0.5) (layer F.Cu) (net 16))
 (segment (start 145.604 74.295) (end 147.382 76.073) (width 0.5) (layer F.Cu) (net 16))
 (segment (start 142.21 74.295) (end 145.604 74.295) (width 0.5) (layer F.Cu) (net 16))
 (segment (start 133.485999 75.591895) (end 133.485999 78.875999) (width 0.5) (layer B.Cu) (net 6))
 (segment (start 133.728894 75.349) (end 133.485999 75.591895) (width 0.5) (layer B.Cu) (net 6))
 (segment (start 134.436 75.349) (end 133.728894 75.349) (width 0.5) (layer B.Cu) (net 6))
 (via (at 140.462 82.55) (size 0.8) (drill 0.4) (layers F.Cu B.Cu) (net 6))
 (segment (start 137.16 82.55) (end 140.462 82.55) (width 0.5) (layer B.Cu) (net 6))
 (segment (start 133.485999 78.875999) (end 137.16 82.55) (width 0.5) (layer B.Cu) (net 6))
 (segment (start 142.305 82.55) (end 142.432 82.423) (width 0.5) (layer F.Cu) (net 6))
 (segment (start 140.462 82.55) (end 142.305 82.55) (width 0.5) (layer F.Cu) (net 6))
 (segment (start 136.601 76.149) (end 135.636 76.149) (width 0.5) (layer B.Cu) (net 5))
 (segment (start 137.668 77.216) (end 136.601 76.149) (width 0.5) (layer B.Cu) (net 5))
 (via (at 144.272 81.026) (size 0.8) (drill 0.4) (layers F.Cu B.Cu) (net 5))
 (segment (start 140.462 77.216) (end 144.272 81.026) (width 0.5) (layer B.Cu) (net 5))
 (segment (start 137.668 77.216) (end 140.462 77.216) (width 0.5) (layer B.Cu) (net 5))
 (segment (start 142.559 81.026) (end 142.432 81.153) (width 0.5) (layer F.Cu) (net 5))
 (segment (start 144.272 81.026) (end 142.559 81.026) (width 0.5) (layer F.Cu) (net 5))
 (segment (start 152.781 83.566) (end 154.149 83.566) (width 0.5) (layer F.Cu) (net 2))
 (segment (start 152.019 84.328) (end 152.781 83.566) (width 0.5) (layer F.Cu) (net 2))
 (via (at 144.399 77.343) (size 0.8) (drill 0.4) (layers F.Cu B.Cu) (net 2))
 (segment (start 144.399 77.343) (end 142.432 77.343) (width 0.5) (layer F.Cu) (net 2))
 (segment (start 144.399 74.168) (end 148.209 70.358) (width 0.5) (layer B.Cu) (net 2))
 (segment (start 144.399 77.343) (end 144.399 74.168) (width 0.5) (layer B.Cu) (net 2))
 (segment (start 148.844 83.566) (end 144.399 79.121) (width 0.5) (layer B.Cu) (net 2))
 (segment (start 155.702 83.566) (end 148.844 83.566) (width 0.5) (layer B.Cu) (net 2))
 (segment (start 154.149 83.566) (end 155.702 83.566) (width 0.5) (layer F.Cu) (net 2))
 (segment (start 144.399 79.121) (end 144.399 77.343) (width 0.5) (layer B.Cu) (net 2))
 (via (at 155.702 83.566) (size 0.8) (drill 0.4) (layers F.Cu B.Cu) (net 2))
 (segment (start 152.527 79.756) (end 152.019 80.264) (width 0.5) (layer F.Cu) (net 3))
 (segment (start 154.149 79.756) (end 152.527 79.756) (width 0.5) (layer F.Cu) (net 3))
 (via (at 156.083 79.883) (size 0.8) (drill 0.4) (layers F.Cu B.Cu) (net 3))
 (segment (start 155.956 79.756) (end 156.083 79.883) (width 0.5) (layer F.Cu) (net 3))
 (segment (start 154.149 79.756) (end 155.956 79.756) (width 0.5) (layer F.Cu) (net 3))
 (segment (start 145.415 78.613) (end 142.432 78.613) (width 0.5) (layer F.Cu) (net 3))
 (segment (start 154.813 78.613) (end 156.083 79.883) (width 0.5) (layer B.Cu) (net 3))
 (segment (start 145.415 78.613) (end 154.813 78.613) (width 0.5) (layer B.Cu) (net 3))
 (via (at 145.415 78.613) (size 0.8) (drill 0.4) (layers F.Cu B.Cu) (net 3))
 (via (at 146.685 73.406) (size 0.8) (drill 0.4) (layers F.Cu B.Cu) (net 3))
 (segment (start 145.415 74.676) (end 146.685 73.406) (width 0.5) (layer B.Cu) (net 3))
 (segment (start 145.415 78.613) (end 145.415 74.676) (width 0.5) (layer B.Cu) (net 3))
 (segment (start 146.685 71.374) (end 145.669 70.358) (width 0.5) (layer F.Cu) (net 3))
 (segment (start 146.685 73.406) (end 146.685 71.374) (width 0.5) (layer F.Cu) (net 3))
 (segment (start 163.479 77.246) (end 163.449 77.216) (width 0.5) (layer F.Cu) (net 17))
 (segment (start 165.862 77.246) (end 163.479 77.246) (width 0.5) (layer F.Cu) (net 17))
 (via (at 166.624 75.819) (size 0.8) (drill 0.4) (layers F.Cu B.Cu) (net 17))
 (segment (start 164.592 73.787) (end 166.624 75.819) (width 0.5) (layer B.Cu) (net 17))
 (segment (start 162.433 73.787) (end 164.592 73.787) (width 0.5) (layer B.Cu) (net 17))
 (segment (start 166.624 76.484) (end 165.862 77.246) (width 0.5) (layer F.Cu) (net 17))
 (segment (start 166.624 75.819) (end 166.624 76.484) (width 0.5) (layer F.Cu) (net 17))
 (segment (start 165.64 83.566) (end 165.64 85.82) (width 0.5) (layer F.Cu) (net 18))
 (segment (start 165.354 86.106) (end 163.449 86.106) (width 0.5) (layer F.Cu) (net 18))
 (segment (start 165.64 85.82) (end 165.354 86.106) (width 0.5) (layer F.Cu) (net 18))
 (segment (start 165.227 78.486) (end 165.862 79.121) (width 0.5) (layer F.Cu) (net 18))
 (segment (start 163.449 78.486) (end 165.227 78.486) (width 0.5) (layer F.Cu) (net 18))
 (via (at 165.989 80.391) (size 0.8) (drill 0.4) (layers F.Cu B.Cu) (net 18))
 (segment (start 165.862 80.264) (end 165.989 80.391) (width 0.5) (layer F.Cu) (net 18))
 (segment (start 165.862 79.121) (end 165.862 80.264) (width 0.5) (layer F.Cu) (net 18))
 (via (at 165.64 85.82) (size 0.8) (drill 0.4) (layers F.Cu B.Cu) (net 18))
 (segment (start 165.989 85.471) (end 165.64 85.82) (width 0.5) (layer B.Cu) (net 18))
 (segment (start 165.989 80.391) (end 165.989 85.471) (width 0.5) (layer B.Cu) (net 18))
 (via (at 165.354 75.946) (size 0.8) (drill 0.4) (layers F.Cu B.Cu) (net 18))
 (segment (start 165.989 76.581) (end 165.354 75.946) (width 0.5) (layer B.Cu) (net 18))
 (segment (start 165.989 80.391) (end 165.989 76.581) (width 0.5) (layer B.Cu) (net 18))
 (segment (start 165.354 73.631) (end 165.513 73.472) (width 0.5) (layer F.Cu) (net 18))
 (segment (start 165.354 75.946) (end 165.354 73.631) (width 0.5) (layer F.Cu) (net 18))
 (segment (start 159.893 75.187) (end 159.893 73.787) (width 0.5) (layer B.Cu) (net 18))
 (segment (start 160.652 75.946) (end 159.893 75.187) (width 0.5) (layer B.Cu) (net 18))
 (segment (start 165.354 75.946) (end 160.652 75.946) (width 0.5) (layer B.Cu) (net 18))
 (segment (start 150.144 82.296) (end 150.144 84.328) (width 0.5) (layer F.Cu) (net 27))
 (segment (start 149.658473 80.749527) (end 150.144 80.264) (width 0.5) (layer F.Cu) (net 28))
 (segment (start 149.20649 81.20151) (end 149.658473 80.749527) (width 0.5) (layer F.Cu) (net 28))
 (segment (start 149.20649 85.50099) (end 149.20649 81.20151) (width 0.5) (layer F.Cu) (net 28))
 (segment (start 150.0655 86.36) (end 149.20649 85.50099) (width 0.5) (layer F.Cu) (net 28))
 (segment (start 168.349 70.786) (end 167.513 71.622) (width 0.5) (layer F.Cu) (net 24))
 (segment (start 172.085 70.786) (end 168.349 70.786) (width 0.5) (layer F.Cu) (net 24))
 (segment (start 167.513 72.009) (end 165.1 72.009) (width 0.5) (layer F.Cu) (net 24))
 (segment (start 167.513 71.622) (end 167.513 72.009) (width 0.5) (layer F.Cu) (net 24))
 (segment (start 167.513 72.009) (end 167.513 72.522) (width 0.5) (layer F.Cu) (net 24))
 (segment (start 165.1 72.009) (end 163.83 73.279) (width 0.5) (layer F.Cu) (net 24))
 (segment (start 163.83 73.279) (end 163.83 74.549) (width 0.5) (layer F.Cu) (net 24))
 (segment (start 163.83 74.549) (end 161.671 76.708) (width 0.5) (layer F.Cu) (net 24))
 (segment (start 161.671 76.708) (end 161.671 79.502) (width 0.5) (layer F.Cu) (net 24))
 (segment (start 161.925 79.756) (end 163.449 79.756) (width 0.5) (layer F.Cu) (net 24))
 (segment (start 161.671 79.502) (end 161.925 79.756) (width 0.5) (layer F.Cu) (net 24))
 (segment (start 168.057 75.866) (end 167.513 75.322) (width 0.5) (layer F.Cu) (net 23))
 (segment (start 172.085 75.866) (end 168.057 75.866) (width 0.5) (layer F.Cu) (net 23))
 (segment (start 167.386 74.93) (end 167.513 74.422) (width 0.5) (layer F.Cu) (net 23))
 (segment (start 167.513 75.322) (end 167.386 74.93) (width 0.5) (layer F.Cu) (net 23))
 (segment (start 167.64 75.184) (end 167.386 74.93) (width 0.5) (layer F.Cu) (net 23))
 (segment (start 167.64 80.518) (end 167.64 75.184) (width 0.5) (layer F.Cu) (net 23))
 (segment (start 166.751 81.407) (end 167.64 80.518) (width 0.5) (layer F.Cu) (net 23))
 (segment (start 165.1 81.407) (end 166.751 81.407) (width 0.5) (layer F.Cu) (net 23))
 (segment (start 164.719 81.026) (end 165.1 81.407) (width 0.5) (layer F.Cu) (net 23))
 (segment (start 163.449 81.026) (end 164.719 81.026) (width 0.5) (layer F.Cu) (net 23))
 (segment (start 170.387944 85.866) (end 172.085 85.866) (width 0.5) (layer F.Cu) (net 21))
 (segment (start 168.09 85.866) (end 170.387944 85.866) (width 0.5) (layer F.Cu) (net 21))
 (segment (start 167.64 85.416) (end 168.09 85.866) (width 0.5) (layer F.Cu) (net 21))
 (segment (start 167.64 84.516) (end 167.64 85.416) (width 0.5) (layer F.Cu) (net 21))
 (segment (start 167.64 85.416) (end 165.807 87.249) (width 0.5) (layer F.Cu) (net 21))
 (segment (start 165.807 87.249) (end 161.417 87.249) (width 0.5) (layer F.Cu) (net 21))
 (segment (start 161.417 84.573) (end 162.424 83.566) (width 0.5) (layer F.Cu) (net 21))
 (segment (start 162.424 83.566) (end 163.449 83.566) (width 0.5) (layer F.Cu) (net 21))
 (segment (start 161.417 87.249) (end 161.417 84.573) (width 0.5) (layer F.Cu) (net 21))
 (segment (start 167.32 82.296) (end 167.64 82.616) (width 0.5) (layer F.Cu) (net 22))
 (segment (start 163.449 82.296) (end 167.32 82.296) (width 0.5) (layer F.Cu) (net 22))
 (segment (start 167.64 81.716) (end 167.64 82.616) (width 0.5) (layer F.Cu) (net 22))
 (segment (start 168.49 80.866) (end 167.64 81.716) (width 0.5) (layer F.Cu) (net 22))
 (segment (start 172.085 80.866) (end 168.49 80.866) (width 0.5) (layer F.Cu) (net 22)))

